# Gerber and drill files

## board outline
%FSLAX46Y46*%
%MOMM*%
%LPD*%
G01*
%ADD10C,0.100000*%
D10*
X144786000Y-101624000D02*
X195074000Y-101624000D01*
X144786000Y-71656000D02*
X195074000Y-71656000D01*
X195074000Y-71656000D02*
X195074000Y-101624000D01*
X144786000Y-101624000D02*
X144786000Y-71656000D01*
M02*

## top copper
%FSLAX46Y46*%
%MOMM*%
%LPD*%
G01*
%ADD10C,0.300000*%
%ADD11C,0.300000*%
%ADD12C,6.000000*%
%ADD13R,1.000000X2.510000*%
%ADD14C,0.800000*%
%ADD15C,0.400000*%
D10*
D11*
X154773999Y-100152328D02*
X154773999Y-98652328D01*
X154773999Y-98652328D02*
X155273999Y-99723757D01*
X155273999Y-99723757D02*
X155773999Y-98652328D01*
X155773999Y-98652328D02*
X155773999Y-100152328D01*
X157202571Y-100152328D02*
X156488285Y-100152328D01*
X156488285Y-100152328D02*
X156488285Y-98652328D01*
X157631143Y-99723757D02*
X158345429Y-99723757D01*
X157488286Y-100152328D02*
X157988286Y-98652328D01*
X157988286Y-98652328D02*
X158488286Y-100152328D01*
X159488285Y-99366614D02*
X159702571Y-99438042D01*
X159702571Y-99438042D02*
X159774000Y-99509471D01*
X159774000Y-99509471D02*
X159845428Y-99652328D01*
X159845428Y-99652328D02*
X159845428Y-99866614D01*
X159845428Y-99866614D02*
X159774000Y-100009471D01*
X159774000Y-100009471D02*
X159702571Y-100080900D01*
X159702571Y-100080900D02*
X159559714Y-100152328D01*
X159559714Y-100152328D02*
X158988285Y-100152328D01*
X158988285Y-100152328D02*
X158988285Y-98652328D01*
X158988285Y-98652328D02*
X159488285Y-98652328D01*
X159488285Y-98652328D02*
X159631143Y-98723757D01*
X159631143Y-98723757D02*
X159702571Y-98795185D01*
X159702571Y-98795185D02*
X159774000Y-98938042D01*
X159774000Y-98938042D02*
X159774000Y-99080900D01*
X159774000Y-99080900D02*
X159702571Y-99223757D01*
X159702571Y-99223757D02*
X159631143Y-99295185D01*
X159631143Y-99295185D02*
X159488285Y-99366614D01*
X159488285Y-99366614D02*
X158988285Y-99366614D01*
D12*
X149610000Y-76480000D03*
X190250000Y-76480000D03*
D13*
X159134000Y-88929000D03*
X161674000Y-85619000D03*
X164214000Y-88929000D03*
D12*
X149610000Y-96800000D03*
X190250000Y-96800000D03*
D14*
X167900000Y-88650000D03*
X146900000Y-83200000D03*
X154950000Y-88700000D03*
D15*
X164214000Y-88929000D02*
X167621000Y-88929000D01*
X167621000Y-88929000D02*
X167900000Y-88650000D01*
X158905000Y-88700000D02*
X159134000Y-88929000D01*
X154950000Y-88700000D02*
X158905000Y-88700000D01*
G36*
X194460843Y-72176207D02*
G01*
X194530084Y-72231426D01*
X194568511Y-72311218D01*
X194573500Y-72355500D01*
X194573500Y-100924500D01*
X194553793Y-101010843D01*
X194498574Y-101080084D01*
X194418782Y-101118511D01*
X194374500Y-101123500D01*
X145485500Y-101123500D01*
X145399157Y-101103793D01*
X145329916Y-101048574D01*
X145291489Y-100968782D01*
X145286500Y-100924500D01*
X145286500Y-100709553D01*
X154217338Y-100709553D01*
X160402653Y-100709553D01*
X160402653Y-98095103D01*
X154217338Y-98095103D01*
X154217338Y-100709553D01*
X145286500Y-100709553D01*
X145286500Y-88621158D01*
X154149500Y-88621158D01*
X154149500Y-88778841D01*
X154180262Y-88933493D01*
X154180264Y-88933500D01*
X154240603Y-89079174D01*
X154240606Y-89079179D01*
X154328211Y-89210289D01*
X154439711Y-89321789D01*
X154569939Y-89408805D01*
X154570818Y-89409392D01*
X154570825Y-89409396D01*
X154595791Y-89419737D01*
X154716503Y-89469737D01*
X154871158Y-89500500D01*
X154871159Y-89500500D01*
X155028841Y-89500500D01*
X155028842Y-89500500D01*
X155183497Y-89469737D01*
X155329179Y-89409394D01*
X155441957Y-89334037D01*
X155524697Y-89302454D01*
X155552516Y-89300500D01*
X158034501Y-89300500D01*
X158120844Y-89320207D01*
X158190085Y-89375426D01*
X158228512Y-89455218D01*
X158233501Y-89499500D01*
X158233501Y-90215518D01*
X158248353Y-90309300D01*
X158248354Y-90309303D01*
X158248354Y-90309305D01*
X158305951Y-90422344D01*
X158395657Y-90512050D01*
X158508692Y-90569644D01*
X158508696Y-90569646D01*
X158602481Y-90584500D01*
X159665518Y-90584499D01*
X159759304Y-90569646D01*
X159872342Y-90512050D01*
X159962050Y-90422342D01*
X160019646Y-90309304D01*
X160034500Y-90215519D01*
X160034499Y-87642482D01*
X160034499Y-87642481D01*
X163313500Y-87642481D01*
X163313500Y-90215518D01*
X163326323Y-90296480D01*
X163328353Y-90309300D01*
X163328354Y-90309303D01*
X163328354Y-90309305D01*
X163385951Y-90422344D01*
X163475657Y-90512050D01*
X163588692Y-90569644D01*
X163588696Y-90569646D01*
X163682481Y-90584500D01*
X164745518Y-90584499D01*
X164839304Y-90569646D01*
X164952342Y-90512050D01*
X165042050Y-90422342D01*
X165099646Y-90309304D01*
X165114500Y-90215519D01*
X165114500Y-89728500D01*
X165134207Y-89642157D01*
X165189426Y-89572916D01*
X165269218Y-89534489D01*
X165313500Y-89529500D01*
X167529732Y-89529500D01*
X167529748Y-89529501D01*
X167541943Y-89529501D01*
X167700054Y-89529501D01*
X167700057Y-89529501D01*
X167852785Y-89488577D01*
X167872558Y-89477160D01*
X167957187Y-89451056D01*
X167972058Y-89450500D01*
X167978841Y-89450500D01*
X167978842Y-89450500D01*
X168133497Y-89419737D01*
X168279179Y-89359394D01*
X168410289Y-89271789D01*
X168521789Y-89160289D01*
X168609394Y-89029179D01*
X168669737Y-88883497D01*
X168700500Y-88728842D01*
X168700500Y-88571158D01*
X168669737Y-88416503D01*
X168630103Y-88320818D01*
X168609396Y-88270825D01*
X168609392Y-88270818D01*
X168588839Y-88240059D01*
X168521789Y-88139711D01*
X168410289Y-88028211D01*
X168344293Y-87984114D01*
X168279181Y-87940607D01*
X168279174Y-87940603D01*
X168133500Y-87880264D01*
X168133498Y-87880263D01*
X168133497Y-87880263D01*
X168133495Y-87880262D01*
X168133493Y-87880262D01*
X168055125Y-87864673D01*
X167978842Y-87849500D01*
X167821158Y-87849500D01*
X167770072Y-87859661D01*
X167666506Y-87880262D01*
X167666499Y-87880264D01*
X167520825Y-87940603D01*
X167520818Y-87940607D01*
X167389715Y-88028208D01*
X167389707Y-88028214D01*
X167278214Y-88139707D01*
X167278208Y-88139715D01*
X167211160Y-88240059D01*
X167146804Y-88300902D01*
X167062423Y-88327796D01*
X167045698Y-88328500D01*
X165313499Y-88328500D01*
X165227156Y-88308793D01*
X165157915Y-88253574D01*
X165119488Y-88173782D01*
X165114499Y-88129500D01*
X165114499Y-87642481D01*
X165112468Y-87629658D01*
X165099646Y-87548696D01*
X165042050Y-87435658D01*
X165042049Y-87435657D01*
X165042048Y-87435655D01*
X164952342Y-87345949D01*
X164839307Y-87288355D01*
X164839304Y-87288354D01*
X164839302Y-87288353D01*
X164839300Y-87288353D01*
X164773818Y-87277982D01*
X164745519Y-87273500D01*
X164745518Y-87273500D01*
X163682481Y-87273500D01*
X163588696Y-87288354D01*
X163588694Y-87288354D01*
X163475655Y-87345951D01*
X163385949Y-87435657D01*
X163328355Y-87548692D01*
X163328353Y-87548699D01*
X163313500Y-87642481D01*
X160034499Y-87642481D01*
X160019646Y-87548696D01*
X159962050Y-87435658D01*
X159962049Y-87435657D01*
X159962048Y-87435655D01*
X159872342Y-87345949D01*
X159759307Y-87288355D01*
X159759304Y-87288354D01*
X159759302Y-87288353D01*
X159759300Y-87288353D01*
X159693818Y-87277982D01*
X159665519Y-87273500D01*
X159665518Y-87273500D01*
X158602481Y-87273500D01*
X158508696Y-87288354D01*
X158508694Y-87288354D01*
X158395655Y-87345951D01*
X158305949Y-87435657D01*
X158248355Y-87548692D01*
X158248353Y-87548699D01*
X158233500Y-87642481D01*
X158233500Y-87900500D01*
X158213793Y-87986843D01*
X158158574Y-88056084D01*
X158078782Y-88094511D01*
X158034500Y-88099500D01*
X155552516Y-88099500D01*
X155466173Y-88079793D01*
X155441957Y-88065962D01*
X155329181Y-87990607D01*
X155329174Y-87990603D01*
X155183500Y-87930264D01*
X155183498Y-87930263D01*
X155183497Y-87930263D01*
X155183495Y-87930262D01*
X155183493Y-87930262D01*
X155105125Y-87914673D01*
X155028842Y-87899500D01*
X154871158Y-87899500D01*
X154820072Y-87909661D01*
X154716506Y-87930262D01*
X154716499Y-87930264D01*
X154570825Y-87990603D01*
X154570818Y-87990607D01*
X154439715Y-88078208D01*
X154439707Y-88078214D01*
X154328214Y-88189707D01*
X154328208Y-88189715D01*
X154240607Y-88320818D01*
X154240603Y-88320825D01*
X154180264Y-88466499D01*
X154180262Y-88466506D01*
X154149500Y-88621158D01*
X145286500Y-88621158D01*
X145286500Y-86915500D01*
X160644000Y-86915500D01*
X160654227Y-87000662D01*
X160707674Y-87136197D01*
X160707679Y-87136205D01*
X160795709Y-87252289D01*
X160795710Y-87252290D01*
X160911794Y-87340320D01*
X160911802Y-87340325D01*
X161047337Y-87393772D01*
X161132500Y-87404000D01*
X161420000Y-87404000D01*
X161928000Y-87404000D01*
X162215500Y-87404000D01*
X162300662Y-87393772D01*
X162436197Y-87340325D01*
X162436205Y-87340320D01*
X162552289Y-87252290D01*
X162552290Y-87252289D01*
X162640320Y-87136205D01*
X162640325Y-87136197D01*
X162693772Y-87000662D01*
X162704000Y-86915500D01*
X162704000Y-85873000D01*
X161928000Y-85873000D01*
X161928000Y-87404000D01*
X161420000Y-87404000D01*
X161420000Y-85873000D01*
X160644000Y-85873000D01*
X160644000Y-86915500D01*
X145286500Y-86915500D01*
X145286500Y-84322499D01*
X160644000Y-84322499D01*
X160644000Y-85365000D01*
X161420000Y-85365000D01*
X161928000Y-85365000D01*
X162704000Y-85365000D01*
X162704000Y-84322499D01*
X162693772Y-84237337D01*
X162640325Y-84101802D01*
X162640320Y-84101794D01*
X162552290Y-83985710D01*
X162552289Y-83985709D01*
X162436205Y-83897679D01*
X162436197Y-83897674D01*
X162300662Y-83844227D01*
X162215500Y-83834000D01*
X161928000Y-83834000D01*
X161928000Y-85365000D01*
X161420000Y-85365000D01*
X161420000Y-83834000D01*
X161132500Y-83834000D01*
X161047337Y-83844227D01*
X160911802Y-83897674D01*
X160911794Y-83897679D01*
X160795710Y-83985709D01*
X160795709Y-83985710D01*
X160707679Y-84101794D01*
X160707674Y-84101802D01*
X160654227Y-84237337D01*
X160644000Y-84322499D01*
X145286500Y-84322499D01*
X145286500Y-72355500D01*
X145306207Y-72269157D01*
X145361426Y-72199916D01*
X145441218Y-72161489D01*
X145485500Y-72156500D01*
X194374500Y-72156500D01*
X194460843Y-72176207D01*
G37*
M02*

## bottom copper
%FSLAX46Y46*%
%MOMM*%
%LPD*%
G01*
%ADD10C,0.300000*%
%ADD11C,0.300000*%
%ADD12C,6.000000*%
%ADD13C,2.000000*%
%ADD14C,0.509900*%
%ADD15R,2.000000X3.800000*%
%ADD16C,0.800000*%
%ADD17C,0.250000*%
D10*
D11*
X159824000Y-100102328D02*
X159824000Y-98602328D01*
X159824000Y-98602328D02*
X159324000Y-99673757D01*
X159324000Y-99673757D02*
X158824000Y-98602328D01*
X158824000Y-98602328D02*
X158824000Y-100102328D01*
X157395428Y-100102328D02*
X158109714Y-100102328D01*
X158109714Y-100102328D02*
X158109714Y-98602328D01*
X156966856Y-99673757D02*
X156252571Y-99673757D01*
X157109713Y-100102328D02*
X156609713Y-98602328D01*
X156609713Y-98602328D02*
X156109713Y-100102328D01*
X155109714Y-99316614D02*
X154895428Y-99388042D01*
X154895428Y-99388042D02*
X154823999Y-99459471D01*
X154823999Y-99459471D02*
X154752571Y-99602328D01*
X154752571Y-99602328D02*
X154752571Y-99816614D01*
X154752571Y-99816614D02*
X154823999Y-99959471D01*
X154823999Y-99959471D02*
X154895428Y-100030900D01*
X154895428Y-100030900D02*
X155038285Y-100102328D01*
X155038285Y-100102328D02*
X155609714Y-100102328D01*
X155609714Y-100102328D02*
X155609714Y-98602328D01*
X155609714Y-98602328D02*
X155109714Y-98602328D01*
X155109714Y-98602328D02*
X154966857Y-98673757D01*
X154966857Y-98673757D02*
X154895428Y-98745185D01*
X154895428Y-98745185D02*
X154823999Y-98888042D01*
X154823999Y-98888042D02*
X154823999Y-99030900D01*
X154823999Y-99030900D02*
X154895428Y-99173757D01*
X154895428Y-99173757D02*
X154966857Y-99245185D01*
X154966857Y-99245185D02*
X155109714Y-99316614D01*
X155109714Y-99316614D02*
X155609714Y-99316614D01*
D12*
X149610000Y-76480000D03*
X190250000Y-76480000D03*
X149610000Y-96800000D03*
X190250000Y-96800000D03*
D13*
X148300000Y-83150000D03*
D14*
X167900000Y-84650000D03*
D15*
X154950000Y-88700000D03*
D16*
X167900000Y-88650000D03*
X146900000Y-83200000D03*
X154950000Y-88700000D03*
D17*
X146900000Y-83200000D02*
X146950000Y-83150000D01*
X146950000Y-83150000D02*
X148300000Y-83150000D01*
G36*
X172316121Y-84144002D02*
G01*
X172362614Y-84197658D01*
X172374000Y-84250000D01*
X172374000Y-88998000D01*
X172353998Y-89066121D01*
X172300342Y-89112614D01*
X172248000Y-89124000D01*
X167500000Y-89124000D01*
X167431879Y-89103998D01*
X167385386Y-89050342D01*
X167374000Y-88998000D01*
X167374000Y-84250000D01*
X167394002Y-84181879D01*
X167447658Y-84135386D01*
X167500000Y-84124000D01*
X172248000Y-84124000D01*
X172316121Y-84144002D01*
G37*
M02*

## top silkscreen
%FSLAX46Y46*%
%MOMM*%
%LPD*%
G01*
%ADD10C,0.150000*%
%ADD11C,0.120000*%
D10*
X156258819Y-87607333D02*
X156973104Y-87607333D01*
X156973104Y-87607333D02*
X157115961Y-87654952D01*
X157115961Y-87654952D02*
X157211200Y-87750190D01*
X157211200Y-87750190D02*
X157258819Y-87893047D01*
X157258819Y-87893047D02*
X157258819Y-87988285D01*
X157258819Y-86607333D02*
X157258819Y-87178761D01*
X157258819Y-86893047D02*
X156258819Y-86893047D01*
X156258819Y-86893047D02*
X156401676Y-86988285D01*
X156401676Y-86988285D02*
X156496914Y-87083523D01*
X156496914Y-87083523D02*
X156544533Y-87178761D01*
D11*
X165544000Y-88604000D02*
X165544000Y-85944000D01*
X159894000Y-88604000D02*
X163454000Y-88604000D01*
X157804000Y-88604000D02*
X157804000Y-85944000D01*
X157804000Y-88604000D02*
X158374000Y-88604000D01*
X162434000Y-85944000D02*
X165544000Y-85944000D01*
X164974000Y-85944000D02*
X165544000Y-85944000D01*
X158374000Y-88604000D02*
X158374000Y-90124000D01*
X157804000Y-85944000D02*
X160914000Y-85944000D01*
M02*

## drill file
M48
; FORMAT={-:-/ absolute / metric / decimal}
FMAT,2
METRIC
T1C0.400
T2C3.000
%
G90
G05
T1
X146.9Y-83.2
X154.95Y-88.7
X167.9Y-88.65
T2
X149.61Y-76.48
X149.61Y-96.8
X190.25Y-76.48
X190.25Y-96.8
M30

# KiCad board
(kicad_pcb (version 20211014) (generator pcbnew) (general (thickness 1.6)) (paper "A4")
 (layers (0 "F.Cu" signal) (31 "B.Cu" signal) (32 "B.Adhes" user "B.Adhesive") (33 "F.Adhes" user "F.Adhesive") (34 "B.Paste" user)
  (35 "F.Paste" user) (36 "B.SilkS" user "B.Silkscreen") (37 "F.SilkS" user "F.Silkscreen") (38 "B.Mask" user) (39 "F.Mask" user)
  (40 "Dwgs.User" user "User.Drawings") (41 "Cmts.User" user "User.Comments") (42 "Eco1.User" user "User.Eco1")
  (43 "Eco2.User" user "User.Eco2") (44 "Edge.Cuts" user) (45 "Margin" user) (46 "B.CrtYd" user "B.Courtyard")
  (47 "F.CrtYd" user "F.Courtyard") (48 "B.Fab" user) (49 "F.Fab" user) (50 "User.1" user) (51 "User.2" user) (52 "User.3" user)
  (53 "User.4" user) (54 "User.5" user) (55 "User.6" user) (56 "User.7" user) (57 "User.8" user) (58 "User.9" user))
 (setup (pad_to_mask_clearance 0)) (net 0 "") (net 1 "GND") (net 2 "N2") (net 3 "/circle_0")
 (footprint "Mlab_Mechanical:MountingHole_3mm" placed (layer "F.Cu") (at 149.61 76.48)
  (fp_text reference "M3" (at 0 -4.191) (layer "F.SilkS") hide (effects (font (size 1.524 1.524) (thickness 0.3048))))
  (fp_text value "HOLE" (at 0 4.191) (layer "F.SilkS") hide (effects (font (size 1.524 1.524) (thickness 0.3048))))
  (pad "1" thru_hole circle (at 0 0) (size 6 6) (drill 3) (layers *.Cu *.Mask) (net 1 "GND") (clearance 1) (zone_connect 2)))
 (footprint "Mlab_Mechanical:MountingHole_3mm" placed (layer "F.Cu") (at 190.25 76.48)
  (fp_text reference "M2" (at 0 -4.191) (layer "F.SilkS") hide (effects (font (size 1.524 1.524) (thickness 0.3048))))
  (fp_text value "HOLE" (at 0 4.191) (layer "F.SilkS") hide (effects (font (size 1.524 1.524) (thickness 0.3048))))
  (pad "1" thru_hole circle (at 0 0) (size 6 6) (drill 3) (layers *.Cu *.Mask) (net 1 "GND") (clearance 1) (zone_connect 2)))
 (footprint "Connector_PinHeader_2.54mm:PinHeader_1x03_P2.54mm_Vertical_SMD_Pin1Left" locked (layer "F.Cu") (at 161.674 87.274 90)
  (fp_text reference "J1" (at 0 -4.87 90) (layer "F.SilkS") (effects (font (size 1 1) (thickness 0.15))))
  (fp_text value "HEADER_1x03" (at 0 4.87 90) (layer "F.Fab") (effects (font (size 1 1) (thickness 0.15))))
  (fp_line (start -1.33 3.87) (end 1.33 3.87) (layer "F.SilkS") (width 0.12))
  (fp_line (start -1.33 -1.78) (end -1.33 1.78) (layer "F.SilkS") (width 0.12))
  (fp_line (start -1.33 -3.87) (end 1.33 -3.87) (layer "F.SilkS") (width 0.12))
  (fp_line (start -1.33 -3.87) (end -1.33 -3.3) (layer "F.SilkS") (width 0.12))
  (fp_line (start 1.33 0.76) (end 1.33 3.87) (layer "F.SilkS") (width 0.12))
  (fp_line (start 1.33 3.3) (end 1.33 3.87) (layer "F.SilkS") (width 0.12))
  (fp_line (start -1.33 -3.3) (end -2.85 -3.3) (layer "F.SilkS") (width 0.12))
  (fp_line (start 1.33 -3.87) (end 1.33 -0.76) (layer "F.SilkS") (width 0.12))
  (pad "1" smd rect locked (at -1.655 -2.54 90) (size 2.51 1) (layers "F.Cu" "F.Paste" "F.Mask") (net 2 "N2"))
  (pad "2" smd rect locked (at 1.655 0 90) (size 2.51 1) (layers "F.Cu" "F.Paste" "F.Mask") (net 1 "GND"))
  (pad "3" smd rect locked (at -1.655 2.54 90) (size 2.51 1) (layers "F.Cu" "F.Paste" "F.Mask") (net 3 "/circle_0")))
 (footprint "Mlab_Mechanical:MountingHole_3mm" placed (layer "F.Cu") (at 149.61 96.8)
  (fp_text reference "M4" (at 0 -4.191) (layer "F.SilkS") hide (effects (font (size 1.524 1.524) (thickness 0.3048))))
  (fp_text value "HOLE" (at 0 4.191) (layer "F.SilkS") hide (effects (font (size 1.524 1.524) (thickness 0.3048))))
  (pad "1" thru_hole circle (at 0 0) (size 6 6) (drill 3) (layers *.Cu *.Mask) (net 1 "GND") (clearance 1) (zone_connect 2)))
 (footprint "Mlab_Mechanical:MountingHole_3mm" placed (layer "F.Cu") (at 190.25 96.8)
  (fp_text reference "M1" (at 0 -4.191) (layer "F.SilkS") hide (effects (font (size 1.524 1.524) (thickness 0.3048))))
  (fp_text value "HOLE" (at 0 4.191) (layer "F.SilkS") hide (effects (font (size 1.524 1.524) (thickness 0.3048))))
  (pad "1" thru_hole circle (at 0 0) (size 6 6) (drill 3) (layers *.Cu *.Mask) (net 1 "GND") (clearance 1) (zone_connect 2)))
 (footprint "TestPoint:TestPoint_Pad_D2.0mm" (layer "B.Cu") (at 148.3 83.15 180) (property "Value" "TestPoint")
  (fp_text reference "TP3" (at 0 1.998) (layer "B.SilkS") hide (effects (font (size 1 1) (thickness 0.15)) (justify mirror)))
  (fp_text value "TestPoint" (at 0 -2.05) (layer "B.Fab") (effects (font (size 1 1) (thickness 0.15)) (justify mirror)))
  (pad "1" smd circle (at 0 0 180) (size 2 2) (layers "B.Cu" "B.Mask") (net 1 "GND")))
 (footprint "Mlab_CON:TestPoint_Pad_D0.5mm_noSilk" (layer "B.Cu") (at 167.9 84.65 180) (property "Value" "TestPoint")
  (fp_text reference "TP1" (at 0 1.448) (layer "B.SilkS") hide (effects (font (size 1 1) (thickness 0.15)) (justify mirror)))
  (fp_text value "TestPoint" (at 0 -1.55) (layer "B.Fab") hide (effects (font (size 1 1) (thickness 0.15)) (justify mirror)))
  (pad "1" smd circle (at 0 0 180) (size 0.5099 0.5099) (layers "B.Cu" "B.Mask") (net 3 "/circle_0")))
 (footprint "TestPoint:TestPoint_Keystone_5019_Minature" (layer "B.Cu") (at 154.95 88.7 90) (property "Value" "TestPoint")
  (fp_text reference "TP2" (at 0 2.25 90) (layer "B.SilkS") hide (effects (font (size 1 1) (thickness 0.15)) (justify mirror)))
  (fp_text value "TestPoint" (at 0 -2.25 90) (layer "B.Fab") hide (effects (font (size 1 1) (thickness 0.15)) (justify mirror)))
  (pad "1" smd rect (at 0 0 90) (size 3.8 2) (layers "B.Cu" "B.Paste" "B.Mask") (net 2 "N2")))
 (gr_line (start 144.786 101.624) (end 195.074 101.624) (layer "Edge.Cuts") (width 0.1))
 (gr_line (start 144.786 71.656) (end 195.074 71.656) (layer "Edge.Cuts") (width 0.1))
 (gr_line (start 195.074 71.656) (end 195.074 101.624) (layer "Edge.Cuts") (width 0.1))
 (gr_line (start 144.786 101.624) (end 144.786 71.656) (layer "Edge.Cuts") (width 0.1))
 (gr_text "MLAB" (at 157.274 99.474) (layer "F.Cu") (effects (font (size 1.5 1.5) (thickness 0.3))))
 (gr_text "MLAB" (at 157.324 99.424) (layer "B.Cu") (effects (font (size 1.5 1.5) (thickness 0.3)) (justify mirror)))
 (segment (start 164.214 88.929) (end 167.621 88.929) (width 0.4) (layer "F.Cu") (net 3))
 (segment (start 167.621 88.929) (end 167.9 88.65) (width 0.4) (layer "F.Cu") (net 3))
 (via (at 167.9 88.65) (size 0.8) (drill 0.4) (layers "F.Cu" "B.Cu") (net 3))
 (via (at 146.9 83.2) (size 0.8) (drill 0.4) (layers "F.Cu" "B.Cu") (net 1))
 (segment (start 146.9 83.2) (end 146.95 83.15) (width 0.25) (layer "B.Cu") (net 1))
 (segment (start 146.95 83.15) (end 148.3 83.15) (width 0.25) (layer "B.Cu") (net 1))
 (segment (start 158.905 88.7) (end 159.134 88.929) (width 0.4) (layer "F.Cu") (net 2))
 (segment (start 154.95 88.7) (end 158.905 88.7) (width 0.4) (layer "F.Cu") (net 2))
 (via (at 154.95 88.7) (size 0.8) (drill 0.4) (layers "F.Cu" "B.Cu") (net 2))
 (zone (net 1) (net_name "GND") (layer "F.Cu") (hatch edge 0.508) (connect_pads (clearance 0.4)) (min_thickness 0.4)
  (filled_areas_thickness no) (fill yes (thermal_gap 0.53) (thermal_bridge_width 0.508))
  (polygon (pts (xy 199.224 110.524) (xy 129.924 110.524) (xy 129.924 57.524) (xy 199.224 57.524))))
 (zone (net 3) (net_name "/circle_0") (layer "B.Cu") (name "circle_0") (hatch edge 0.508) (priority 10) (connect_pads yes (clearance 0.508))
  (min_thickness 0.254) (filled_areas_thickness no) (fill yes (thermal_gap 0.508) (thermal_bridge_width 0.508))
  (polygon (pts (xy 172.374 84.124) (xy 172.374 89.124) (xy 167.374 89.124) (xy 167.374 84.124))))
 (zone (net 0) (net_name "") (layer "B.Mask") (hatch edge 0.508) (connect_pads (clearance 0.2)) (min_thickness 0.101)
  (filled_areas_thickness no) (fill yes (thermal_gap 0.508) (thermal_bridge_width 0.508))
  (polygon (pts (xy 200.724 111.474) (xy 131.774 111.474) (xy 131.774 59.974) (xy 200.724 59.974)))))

